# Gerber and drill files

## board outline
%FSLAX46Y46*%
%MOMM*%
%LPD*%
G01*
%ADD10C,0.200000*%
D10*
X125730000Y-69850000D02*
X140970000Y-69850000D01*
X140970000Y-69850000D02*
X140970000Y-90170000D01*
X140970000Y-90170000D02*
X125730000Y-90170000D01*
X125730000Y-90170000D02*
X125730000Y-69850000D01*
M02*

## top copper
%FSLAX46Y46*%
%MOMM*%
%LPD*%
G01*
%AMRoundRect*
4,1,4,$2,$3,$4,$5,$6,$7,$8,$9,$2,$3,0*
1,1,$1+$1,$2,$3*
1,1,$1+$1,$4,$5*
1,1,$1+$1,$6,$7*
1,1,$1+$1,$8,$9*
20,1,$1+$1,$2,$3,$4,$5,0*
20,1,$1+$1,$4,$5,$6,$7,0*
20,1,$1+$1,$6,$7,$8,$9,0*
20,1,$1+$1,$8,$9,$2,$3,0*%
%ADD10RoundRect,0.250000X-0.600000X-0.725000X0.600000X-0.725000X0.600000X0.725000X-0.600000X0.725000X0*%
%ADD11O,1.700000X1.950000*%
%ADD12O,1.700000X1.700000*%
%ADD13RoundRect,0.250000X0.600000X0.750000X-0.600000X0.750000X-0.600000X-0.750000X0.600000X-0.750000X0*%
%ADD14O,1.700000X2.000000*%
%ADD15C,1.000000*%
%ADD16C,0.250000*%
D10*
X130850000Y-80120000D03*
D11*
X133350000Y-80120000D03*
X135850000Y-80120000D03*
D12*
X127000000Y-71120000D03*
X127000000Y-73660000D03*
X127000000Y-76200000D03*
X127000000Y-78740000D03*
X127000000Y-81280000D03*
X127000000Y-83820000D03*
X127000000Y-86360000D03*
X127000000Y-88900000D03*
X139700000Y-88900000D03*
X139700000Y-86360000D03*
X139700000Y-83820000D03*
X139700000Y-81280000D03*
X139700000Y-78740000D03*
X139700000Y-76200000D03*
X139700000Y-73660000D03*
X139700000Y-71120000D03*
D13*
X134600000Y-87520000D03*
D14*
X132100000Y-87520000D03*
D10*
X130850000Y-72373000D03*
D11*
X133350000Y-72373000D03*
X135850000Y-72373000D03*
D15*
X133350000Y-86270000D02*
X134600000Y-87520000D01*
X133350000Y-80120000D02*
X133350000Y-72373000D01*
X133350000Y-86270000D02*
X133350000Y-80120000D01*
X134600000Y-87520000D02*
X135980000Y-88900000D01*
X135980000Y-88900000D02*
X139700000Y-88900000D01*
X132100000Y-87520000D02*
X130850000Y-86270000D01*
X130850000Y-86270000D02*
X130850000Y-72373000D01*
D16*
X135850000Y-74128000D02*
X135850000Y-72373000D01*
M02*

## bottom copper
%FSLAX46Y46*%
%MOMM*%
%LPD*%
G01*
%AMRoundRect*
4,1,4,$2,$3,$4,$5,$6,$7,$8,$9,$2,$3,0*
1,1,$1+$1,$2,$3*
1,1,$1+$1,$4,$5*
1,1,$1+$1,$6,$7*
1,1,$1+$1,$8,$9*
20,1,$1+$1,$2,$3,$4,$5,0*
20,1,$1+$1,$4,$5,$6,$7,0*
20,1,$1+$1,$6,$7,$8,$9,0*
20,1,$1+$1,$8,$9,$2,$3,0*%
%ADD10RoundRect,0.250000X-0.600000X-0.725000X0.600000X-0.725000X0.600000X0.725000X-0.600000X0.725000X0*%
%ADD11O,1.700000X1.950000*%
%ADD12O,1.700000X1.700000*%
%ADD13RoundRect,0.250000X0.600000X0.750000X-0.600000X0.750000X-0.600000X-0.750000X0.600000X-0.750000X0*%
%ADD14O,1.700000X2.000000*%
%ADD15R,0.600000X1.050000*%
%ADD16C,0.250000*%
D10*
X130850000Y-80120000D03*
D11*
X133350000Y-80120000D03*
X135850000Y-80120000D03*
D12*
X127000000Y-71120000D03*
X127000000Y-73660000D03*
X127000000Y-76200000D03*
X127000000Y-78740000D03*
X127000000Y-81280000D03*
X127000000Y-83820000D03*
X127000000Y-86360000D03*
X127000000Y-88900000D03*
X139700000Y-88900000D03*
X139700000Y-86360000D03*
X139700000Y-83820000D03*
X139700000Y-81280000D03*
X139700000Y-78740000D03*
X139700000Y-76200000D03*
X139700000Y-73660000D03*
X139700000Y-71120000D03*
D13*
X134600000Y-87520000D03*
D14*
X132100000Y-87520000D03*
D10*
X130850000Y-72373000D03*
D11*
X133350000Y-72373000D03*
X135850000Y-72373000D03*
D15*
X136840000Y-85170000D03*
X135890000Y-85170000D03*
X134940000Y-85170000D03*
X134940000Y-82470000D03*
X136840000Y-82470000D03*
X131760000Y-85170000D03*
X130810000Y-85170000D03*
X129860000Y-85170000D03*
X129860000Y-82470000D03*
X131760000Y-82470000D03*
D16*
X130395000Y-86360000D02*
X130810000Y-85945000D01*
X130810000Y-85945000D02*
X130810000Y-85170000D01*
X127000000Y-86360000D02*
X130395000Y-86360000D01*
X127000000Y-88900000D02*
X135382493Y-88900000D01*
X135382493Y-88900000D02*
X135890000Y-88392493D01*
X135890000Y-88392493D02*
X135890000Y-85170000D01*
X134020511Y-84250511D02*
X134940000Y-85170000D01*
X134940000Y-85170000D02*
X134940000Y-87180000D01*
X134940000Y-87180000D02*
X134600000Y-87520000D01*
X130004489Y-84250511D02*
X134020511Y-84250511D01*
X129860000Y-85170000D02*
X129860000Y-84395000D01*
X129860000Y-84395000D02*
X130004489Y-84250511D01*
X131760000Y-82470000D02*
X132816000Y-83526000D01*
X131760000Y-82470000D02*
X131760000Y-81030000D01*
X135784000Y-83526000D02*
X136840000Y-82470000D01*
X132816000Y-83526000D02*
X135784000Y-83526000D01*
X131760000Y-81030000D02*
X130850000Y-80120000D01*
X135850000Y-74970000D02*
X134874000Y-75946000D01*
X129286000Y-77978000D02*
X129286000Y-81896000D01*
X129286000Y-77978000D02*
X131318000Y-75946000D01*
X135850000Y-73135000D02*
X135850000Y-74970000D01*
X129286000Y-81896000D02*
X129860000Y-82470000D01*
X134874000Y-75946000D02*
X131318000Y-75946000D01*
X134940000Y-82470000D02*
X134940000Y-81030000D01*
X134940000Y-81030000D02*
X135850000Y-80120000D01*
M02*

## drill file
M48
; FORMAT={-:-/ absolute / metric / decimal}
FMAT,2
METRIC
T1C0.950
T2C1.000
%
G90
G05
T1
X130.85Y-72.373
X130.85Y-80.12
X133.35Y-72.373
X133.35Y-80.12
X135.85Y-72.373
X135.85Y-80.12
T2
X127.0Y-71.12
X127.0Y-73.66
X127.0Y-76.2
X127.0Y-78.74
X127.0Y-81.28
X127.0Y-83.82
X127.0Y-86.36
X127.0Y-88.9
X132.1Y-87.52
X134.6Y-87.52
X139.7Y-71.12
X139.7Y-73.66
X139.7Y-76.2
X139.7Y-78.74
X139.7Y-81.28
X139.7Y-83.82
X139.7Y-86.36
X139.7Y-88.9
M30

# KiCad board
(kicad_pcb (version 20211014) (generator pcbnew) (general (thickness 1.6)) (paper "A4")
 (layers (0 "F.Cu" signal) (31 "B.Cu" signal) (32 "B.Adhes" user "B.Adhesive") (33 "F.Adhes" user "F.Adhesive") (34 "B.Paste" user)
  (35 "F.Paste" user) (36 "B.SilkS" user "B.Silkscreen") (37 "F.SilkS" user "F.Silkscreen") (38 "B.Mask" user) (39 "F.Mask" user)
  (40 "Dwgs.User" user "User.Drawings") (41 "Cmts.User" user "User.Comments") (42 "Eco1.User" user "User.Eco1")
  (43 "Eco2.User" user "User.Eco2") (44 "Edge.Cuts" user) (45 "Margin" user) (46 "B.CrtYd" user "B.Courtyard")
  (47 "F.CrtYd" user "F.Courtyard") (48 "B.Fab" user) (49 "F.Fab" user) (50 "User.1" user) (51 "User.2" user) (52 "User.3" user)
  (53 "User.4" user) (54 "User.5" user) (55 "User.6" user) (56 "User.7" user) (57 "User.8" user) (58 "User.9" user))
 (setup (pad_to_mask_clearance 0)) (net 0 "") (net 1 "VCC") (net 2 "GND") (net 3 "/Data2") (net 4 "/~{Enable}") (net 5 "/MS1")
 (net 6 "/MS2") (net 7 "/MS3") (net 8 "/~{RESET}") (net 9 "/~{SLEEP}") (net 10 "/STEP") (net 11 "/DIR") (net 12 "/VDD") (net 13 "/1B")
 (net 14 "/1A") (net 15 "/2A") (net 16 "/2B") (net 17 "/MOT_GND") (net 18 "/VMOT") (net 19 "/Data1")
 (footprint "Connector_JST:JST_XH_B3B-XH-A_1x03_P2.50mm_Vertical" (layer "F.Cu") (at 130.85 80.12)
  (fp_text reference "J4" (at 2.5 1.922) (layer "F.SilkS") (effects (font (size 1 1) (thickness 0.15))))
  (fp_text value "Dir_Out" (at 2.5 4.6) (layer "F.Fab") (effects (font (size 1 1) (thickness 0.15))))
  (pad "1" thru_hole roundrect locked (at 0 0) (size 1.7 1.95) (drill 0.95) (layers *.Cu *.Mask) (roundrect_rratio 0.1470588235)
   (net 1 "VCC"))
  (pad "2" thru_hole oval locked (at 2.5 0) (size 1.7 1.95) (drill 0.95) (layers *.Cu *.Mask) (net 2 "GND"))
  (pad "3" thru_hole oval locked (at 5 0) (size 1.7 1.95) (drill 0.95) (layers *.Cu *.Mask) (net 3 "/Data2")))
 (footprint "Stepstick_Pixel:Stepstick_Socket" (layer "F.Cu") (at 133.35 80.01)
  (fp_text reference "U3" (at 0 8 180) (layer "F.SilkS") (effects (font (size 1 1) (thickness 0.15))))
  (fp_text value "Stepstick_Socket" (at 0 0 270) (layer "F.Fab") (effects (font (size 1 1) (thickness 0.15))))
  (pad "1" thru_hole oval (at -6.35 -8.89 270) (size 1.7 1.7) (drill 1) (layers *.Cu *.Mask) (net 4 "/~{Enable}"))
  (pad "2" thru_hole oval (at -6.35 -6.35 270) (size 1.7 1.7) (drill 1) (layers *.Cu *.Mask) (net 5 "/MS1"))
  (pad "3" thru_hole oval (at -6.35 -3.81 270) (size 1.7 1.7) (drill 1) (layers *.Cu *.Mask) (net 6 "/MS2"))
  (pad "4" thru_hole oval (at -6.35 -1.27 270) (size 1.7 1.7) (drill 1) (layers *.Cu *.Mask) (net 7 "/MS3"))
  (pad "5" thru_hole oval (at -6.35 1.27 270) (size 1.7 1.7) (drill 1) (layers *.Cu *.Mask) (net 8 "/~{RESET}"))
  (pad "6" thru_hole oval (at -6.35 3.81 270) (size 1.7 1.7) (drill 1) (layers *.Cu *.Mask) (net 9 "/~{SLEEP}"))
  (pad "7" thru_hole oval (at -6.35 6.35 270) (size 1.7 1.7) (drill 1) (layers *.Cu *.Mask) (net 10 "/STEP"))
  (pad "8" thru_hole oval (at -6.35 8.89 270) (size 1.7 1.7) (drill 1) (layers *.Cu *.Mask) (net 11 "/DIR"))
  (pad "9" thru_hole oval (at 6.35 8.89 270) (size 1.7 1.7) (drill 1) (layers *.Cu *.Mask) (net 2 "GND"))
  (pad "10" thru_hole oval (at 6.35 6.35 270) (size 1.7 1.7) (drill 1) (layers *.Cu *.Mask) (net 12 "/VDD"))
  (pad "11" thru_hole oval (at 6.35 3.81 270) (size 1.7 1.7) (drill 1) (layers *.Cu *.Mask) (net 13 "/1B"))
  (pad "12" thru_hole oval (at 6.35 1.27 270) (size 1.7 1.7) (drill 1) (layers *.Cu *.Mask) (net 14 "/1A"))
  (pad "13" thru_hole oval (at 6.35 -1.27 270) (size 1.7 1.7) (drill 1) (layers *.Cu *.Mask) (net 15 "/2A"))
  (pad "14" thru_hole oval (at 6.35 -3.81 270) (size 1.7 1.7) (drill 1) (layers *.Cu *.Mask) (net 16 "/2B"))
  (pad "15" thru_hole oval (at 6.35 -6.35 270) (size 1.7 1.7) (drill 1) (layers *.Cu *.Mask) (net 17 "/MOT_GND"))
  (pad "16" thru_hole oval (at 6.35 -8.89 270) (size 1.7 1.7) (drill 1) (layers *.Cu *.Mask) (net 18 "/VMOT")))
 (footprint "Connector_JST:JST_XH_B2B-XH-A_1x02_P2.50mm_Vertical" (layer "F.Cu") (at 134.6 87.52 180)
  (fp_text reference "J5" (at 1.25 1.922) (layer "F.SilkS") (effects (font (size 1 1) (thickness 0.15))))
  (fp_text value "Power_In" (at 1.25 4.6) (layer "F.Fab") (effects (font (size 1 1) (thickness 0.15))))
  (pad "1" thru_hole roundrect locked (at 0 0 180) (size 1.7 2) (drill 1) (layers *.Cu *.Mask) (roundrect_rratio 0.1470588235) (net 2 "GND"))
  (pad "2" thru_hole oval locked (at 2.5 0 180) (size 1.7 2) (drill 1) (layers *.Cu *.Mask) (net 1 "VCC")))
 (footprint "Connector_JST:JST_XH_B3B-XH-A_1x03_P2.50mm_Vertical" (layer "F.Cu") (at 130.85 72.373)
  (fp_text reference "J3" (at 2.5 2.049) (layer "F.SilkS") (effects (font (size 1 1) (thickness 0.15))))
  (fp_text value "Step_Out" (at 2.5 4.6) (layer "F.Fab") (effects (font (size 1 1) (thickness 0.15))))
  (pad "1" thru_hole roundrect locked (at 0 0) (size 1.7 1.95) (drill 0.95) (layers *.Cu *.Mask) (roundrect_rratio 0.1470588235)
   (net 1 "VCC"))
  (pad "2" thru_hole oval locked (at 2.5 0) (size 1.7 1.95) (drill 0.95) (layers *.Cu *.Mask) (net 2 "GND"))
  (pad "3" thru_hole oval locked (at 5 0) (size 1.7 1.95) (drill 0.95) (layers *.Cu *.Mask) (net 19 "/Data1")))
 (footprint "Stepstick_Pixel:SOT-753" (layer "B.Cu") (at 135.89 83.82 180)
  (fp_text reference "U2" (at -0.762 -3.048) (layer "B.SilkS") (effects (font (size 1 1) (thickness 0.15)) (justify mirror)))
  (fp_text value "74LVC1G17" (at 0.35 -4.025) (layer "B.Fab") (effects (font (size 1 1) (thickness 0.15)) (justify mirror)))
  (pad "1" smd rect (at -0.95 -1.35 180) (size 0.6 1.05) (layers "B.Cu" "B.Paste" "B.Mask") (solder_mask_margin 0.07))
  (pad "2" smd rect (at 0 -1.35 180) (size 0.6 1.05) (layers "B.Cu" "B.Paste" "B.Mask") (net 11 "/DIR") (solder_mask_margin 0.07))
  (pad "3" smd rect (at 0.95 -1.35 180) (size 0.6 1.05) (layers "B.Cu" "B.Paste" "B.Mask") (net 2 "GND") (solder_mask_margin 0.07))
  (pad "4" smd rect (at 0.95 1.35 180) (size 0.6 1.05) (layers "B.Cu" "B.Paste" "B.Mask") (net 3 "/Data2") (solder_mask_margin 0.07))
  (pad "5" smd rect (at -0.95 1.35 180) (size 0.6 1.05) (layers "B.Cu" "B.Paste" "B.Mask") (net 1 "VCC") (solder_mask_margin 0.07)))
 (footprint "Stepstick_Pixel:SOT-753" (layer "B.Cu") (at 130.81 83.82 180)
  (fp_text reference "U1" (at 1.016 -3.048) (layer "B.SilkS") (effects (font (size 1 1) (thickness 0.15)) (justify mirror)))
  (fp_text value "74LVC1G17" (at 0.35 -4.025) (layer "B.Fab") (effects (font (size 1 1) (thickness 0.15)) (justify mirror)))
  (pad "1" smd rect (at -0.95 -1.35 180) (size 0.6 1.05) (layers "B.Cu" "B.Paste" "B.Mask") (solder_mask_margin 0.07))
  (pad "2" smd rect (at 0 -1.35 180) (size 0.6 1.05) (layers "B.Cu" "B.Paste" "B.Mask") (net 10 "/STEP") (solder_mask_margin 0.07))
  (pad "3" smd rect (at 0.95 -1.35 180) (size 0.6 1.05) (layers "B.Cu" "B.Paste" "B.Mask") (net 2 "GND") (solder_mask_margin 0.07))
  (pad "4" smd rect (at 0.95 1.35 180) (size 0.6 1.05) (layers "B.Cu" "B.Paste" "B.Mask") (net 19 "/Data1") (solder_mask_margin 0.07))
  (pad "5" smd rect (at -0.95 1.35 180) (size 0.6 1.05) (layers "B.Cu" "B.Paste" "B.Mask") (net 1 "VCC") (solder_mask_margin 0.07)))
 (gr_line (start 125.73 69.85) (end 140.97 69.85) (layer "Edge.Cuts") (width 0.2))
 (gr_line (start 140.97 69.85) (end 140.97 90.17) (layer "Edge.Cuts") (width 0.2))
 (gr_line (start 140.97 90.17) (end 125.73 90.17) (layer "Edge.Cuts") (width 0.2))
 (gr_line (start 125.73 90.17) (end 125.73 69.85) (layer "Edge.Cuts") (width 0.2))
 (segment (start 130.395 86.36) (end 130.81 85.945) (width 0.25) (layer "B.Cu") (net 10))
 (segment (start 130.81 85.945) (end 130.81 85.17) (width 0.25) (layer "B.Cu") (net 10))
 (segment (start 127 86.36) (end 130.395 86.36) (width 0.25) (layer "B.Cu") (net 10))
 (segment (start 127 88.9) (end 135.382493 88.9) (width 0.25) (layer "B.Cu") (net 11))
 (segment (start 135.382493 88.9) (end 135.89 88.392493) (width 0.25) (layer "B.Cu") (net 11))
 (segment (start 135.89 88.392493) (end 135.89 85.17) (width 0.25) (layer "B.Cu") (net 11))
 (segment (start 133.35 86.27) (end 134.6 87.52) (width 1) (layer "F.Cu") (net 2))
 (segment (start 133.35 80.12) (end 133.35 72.373) (width 1) (layer "F.Cu") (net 2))
 (segment (start 133.35 86.27) (end 133.35 80.12) (width 1) (layer "F.Cu") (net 2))
 (segment (start 134.6 87.52) (end 135.98 88.9) (width 1) (layer "F.Cu") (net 2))
 (segment (start 135.98 88.9) (end 139.7 88.9) (width 1) (layer "F.Cu") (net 2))
 (segment (start 134.020511 84.250511) (end 134.94 85.17) (width 0.25) (layer "B.Cu") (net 2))
 (segment (start 134.94 85.17) (end 134.94 87.18) (width 0.25) (layer "B.Cu") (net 2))
 (segment (start 134.94 87.18) (end 134.6 87.52) (width 0.25) (layer "B.Cu") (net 2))
 (segment (start 130.004489 84.250511) (end 134.020511 84.250511) (width 0.25) (layer "B.Cu") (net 2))
 (segment (start 129.86 85.17) (end 129.86 84.395) (width 0.25) (layer "B.Cu") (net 2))
 (segment (start 129.86 84.395) (end 130.004489 84.250511) (width 0.25) (layer "B.Cu") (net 2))
 (segment (start 132.1 87.52) (end 130.85 86.27) (width 1) (layer "F.Cu") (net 1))
 (segment (start 130.85 86.27) (end 130.85 72.373) (width 1) (layer "F.Cu") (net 1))
 (segment (start 131.76 82.47) (end 132.816 83.526) (width 0.25) (layer "B.Cu") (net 1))
 (segment (start 131.76 82.47) (end 131.76 81.03) (width 0.25) (layer "B.Cu") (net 1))
 (segment (start 135.784 83.526) (end 136.84 82.47) (width 0.25) (layer "B.Cu") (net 1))
 (segment (start 132.816 83.526) (end 135.784 83.526) (width 0.25) (layer "B.Cu") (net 1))
 (segment (start 131.76 81.03) (end 130.85 80.12) (width 0.25) (layer "B.Cu") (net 1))
 (segment (start 135.85 74.128) (end 135.85 72.373) (width 0.25) (layer "F.Cu") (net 19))
 (segment (start 135.85 74.97) (end 134.874 75.946) (width 0.25) (layer "B.Cu") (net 19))
 (segment (start 129.286 77.978) (end 129.286 81.896) (width 0.25) (layer "B.Cu") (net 19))
 (segment (start 129.286 77.978) (end 131.318 75.946) (width 0.25) (layer "B.Cu") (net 19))
 (segment (start 135.85 73.135) (end 135.85 74.97) (width 0.25) (layer "B.Cu") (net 19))
 (segment (start 129.286 81.896) (end 129.86 82.47) (width 0.25) (layer "B.Cu") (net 19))
 (segment (start 134.874 75.946) (end 131.318 75.946) (width 0.25) (layer "B.Cu") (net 19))
 (segment (start 134.94 82.47) (end 134.94 81.03) (width 0.25) (layer "B.Cu") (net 3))
 (segment (start 134.94 81.03) (end 135.85 80.12) (width 0.25) (layer "B.Cu") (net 3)))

